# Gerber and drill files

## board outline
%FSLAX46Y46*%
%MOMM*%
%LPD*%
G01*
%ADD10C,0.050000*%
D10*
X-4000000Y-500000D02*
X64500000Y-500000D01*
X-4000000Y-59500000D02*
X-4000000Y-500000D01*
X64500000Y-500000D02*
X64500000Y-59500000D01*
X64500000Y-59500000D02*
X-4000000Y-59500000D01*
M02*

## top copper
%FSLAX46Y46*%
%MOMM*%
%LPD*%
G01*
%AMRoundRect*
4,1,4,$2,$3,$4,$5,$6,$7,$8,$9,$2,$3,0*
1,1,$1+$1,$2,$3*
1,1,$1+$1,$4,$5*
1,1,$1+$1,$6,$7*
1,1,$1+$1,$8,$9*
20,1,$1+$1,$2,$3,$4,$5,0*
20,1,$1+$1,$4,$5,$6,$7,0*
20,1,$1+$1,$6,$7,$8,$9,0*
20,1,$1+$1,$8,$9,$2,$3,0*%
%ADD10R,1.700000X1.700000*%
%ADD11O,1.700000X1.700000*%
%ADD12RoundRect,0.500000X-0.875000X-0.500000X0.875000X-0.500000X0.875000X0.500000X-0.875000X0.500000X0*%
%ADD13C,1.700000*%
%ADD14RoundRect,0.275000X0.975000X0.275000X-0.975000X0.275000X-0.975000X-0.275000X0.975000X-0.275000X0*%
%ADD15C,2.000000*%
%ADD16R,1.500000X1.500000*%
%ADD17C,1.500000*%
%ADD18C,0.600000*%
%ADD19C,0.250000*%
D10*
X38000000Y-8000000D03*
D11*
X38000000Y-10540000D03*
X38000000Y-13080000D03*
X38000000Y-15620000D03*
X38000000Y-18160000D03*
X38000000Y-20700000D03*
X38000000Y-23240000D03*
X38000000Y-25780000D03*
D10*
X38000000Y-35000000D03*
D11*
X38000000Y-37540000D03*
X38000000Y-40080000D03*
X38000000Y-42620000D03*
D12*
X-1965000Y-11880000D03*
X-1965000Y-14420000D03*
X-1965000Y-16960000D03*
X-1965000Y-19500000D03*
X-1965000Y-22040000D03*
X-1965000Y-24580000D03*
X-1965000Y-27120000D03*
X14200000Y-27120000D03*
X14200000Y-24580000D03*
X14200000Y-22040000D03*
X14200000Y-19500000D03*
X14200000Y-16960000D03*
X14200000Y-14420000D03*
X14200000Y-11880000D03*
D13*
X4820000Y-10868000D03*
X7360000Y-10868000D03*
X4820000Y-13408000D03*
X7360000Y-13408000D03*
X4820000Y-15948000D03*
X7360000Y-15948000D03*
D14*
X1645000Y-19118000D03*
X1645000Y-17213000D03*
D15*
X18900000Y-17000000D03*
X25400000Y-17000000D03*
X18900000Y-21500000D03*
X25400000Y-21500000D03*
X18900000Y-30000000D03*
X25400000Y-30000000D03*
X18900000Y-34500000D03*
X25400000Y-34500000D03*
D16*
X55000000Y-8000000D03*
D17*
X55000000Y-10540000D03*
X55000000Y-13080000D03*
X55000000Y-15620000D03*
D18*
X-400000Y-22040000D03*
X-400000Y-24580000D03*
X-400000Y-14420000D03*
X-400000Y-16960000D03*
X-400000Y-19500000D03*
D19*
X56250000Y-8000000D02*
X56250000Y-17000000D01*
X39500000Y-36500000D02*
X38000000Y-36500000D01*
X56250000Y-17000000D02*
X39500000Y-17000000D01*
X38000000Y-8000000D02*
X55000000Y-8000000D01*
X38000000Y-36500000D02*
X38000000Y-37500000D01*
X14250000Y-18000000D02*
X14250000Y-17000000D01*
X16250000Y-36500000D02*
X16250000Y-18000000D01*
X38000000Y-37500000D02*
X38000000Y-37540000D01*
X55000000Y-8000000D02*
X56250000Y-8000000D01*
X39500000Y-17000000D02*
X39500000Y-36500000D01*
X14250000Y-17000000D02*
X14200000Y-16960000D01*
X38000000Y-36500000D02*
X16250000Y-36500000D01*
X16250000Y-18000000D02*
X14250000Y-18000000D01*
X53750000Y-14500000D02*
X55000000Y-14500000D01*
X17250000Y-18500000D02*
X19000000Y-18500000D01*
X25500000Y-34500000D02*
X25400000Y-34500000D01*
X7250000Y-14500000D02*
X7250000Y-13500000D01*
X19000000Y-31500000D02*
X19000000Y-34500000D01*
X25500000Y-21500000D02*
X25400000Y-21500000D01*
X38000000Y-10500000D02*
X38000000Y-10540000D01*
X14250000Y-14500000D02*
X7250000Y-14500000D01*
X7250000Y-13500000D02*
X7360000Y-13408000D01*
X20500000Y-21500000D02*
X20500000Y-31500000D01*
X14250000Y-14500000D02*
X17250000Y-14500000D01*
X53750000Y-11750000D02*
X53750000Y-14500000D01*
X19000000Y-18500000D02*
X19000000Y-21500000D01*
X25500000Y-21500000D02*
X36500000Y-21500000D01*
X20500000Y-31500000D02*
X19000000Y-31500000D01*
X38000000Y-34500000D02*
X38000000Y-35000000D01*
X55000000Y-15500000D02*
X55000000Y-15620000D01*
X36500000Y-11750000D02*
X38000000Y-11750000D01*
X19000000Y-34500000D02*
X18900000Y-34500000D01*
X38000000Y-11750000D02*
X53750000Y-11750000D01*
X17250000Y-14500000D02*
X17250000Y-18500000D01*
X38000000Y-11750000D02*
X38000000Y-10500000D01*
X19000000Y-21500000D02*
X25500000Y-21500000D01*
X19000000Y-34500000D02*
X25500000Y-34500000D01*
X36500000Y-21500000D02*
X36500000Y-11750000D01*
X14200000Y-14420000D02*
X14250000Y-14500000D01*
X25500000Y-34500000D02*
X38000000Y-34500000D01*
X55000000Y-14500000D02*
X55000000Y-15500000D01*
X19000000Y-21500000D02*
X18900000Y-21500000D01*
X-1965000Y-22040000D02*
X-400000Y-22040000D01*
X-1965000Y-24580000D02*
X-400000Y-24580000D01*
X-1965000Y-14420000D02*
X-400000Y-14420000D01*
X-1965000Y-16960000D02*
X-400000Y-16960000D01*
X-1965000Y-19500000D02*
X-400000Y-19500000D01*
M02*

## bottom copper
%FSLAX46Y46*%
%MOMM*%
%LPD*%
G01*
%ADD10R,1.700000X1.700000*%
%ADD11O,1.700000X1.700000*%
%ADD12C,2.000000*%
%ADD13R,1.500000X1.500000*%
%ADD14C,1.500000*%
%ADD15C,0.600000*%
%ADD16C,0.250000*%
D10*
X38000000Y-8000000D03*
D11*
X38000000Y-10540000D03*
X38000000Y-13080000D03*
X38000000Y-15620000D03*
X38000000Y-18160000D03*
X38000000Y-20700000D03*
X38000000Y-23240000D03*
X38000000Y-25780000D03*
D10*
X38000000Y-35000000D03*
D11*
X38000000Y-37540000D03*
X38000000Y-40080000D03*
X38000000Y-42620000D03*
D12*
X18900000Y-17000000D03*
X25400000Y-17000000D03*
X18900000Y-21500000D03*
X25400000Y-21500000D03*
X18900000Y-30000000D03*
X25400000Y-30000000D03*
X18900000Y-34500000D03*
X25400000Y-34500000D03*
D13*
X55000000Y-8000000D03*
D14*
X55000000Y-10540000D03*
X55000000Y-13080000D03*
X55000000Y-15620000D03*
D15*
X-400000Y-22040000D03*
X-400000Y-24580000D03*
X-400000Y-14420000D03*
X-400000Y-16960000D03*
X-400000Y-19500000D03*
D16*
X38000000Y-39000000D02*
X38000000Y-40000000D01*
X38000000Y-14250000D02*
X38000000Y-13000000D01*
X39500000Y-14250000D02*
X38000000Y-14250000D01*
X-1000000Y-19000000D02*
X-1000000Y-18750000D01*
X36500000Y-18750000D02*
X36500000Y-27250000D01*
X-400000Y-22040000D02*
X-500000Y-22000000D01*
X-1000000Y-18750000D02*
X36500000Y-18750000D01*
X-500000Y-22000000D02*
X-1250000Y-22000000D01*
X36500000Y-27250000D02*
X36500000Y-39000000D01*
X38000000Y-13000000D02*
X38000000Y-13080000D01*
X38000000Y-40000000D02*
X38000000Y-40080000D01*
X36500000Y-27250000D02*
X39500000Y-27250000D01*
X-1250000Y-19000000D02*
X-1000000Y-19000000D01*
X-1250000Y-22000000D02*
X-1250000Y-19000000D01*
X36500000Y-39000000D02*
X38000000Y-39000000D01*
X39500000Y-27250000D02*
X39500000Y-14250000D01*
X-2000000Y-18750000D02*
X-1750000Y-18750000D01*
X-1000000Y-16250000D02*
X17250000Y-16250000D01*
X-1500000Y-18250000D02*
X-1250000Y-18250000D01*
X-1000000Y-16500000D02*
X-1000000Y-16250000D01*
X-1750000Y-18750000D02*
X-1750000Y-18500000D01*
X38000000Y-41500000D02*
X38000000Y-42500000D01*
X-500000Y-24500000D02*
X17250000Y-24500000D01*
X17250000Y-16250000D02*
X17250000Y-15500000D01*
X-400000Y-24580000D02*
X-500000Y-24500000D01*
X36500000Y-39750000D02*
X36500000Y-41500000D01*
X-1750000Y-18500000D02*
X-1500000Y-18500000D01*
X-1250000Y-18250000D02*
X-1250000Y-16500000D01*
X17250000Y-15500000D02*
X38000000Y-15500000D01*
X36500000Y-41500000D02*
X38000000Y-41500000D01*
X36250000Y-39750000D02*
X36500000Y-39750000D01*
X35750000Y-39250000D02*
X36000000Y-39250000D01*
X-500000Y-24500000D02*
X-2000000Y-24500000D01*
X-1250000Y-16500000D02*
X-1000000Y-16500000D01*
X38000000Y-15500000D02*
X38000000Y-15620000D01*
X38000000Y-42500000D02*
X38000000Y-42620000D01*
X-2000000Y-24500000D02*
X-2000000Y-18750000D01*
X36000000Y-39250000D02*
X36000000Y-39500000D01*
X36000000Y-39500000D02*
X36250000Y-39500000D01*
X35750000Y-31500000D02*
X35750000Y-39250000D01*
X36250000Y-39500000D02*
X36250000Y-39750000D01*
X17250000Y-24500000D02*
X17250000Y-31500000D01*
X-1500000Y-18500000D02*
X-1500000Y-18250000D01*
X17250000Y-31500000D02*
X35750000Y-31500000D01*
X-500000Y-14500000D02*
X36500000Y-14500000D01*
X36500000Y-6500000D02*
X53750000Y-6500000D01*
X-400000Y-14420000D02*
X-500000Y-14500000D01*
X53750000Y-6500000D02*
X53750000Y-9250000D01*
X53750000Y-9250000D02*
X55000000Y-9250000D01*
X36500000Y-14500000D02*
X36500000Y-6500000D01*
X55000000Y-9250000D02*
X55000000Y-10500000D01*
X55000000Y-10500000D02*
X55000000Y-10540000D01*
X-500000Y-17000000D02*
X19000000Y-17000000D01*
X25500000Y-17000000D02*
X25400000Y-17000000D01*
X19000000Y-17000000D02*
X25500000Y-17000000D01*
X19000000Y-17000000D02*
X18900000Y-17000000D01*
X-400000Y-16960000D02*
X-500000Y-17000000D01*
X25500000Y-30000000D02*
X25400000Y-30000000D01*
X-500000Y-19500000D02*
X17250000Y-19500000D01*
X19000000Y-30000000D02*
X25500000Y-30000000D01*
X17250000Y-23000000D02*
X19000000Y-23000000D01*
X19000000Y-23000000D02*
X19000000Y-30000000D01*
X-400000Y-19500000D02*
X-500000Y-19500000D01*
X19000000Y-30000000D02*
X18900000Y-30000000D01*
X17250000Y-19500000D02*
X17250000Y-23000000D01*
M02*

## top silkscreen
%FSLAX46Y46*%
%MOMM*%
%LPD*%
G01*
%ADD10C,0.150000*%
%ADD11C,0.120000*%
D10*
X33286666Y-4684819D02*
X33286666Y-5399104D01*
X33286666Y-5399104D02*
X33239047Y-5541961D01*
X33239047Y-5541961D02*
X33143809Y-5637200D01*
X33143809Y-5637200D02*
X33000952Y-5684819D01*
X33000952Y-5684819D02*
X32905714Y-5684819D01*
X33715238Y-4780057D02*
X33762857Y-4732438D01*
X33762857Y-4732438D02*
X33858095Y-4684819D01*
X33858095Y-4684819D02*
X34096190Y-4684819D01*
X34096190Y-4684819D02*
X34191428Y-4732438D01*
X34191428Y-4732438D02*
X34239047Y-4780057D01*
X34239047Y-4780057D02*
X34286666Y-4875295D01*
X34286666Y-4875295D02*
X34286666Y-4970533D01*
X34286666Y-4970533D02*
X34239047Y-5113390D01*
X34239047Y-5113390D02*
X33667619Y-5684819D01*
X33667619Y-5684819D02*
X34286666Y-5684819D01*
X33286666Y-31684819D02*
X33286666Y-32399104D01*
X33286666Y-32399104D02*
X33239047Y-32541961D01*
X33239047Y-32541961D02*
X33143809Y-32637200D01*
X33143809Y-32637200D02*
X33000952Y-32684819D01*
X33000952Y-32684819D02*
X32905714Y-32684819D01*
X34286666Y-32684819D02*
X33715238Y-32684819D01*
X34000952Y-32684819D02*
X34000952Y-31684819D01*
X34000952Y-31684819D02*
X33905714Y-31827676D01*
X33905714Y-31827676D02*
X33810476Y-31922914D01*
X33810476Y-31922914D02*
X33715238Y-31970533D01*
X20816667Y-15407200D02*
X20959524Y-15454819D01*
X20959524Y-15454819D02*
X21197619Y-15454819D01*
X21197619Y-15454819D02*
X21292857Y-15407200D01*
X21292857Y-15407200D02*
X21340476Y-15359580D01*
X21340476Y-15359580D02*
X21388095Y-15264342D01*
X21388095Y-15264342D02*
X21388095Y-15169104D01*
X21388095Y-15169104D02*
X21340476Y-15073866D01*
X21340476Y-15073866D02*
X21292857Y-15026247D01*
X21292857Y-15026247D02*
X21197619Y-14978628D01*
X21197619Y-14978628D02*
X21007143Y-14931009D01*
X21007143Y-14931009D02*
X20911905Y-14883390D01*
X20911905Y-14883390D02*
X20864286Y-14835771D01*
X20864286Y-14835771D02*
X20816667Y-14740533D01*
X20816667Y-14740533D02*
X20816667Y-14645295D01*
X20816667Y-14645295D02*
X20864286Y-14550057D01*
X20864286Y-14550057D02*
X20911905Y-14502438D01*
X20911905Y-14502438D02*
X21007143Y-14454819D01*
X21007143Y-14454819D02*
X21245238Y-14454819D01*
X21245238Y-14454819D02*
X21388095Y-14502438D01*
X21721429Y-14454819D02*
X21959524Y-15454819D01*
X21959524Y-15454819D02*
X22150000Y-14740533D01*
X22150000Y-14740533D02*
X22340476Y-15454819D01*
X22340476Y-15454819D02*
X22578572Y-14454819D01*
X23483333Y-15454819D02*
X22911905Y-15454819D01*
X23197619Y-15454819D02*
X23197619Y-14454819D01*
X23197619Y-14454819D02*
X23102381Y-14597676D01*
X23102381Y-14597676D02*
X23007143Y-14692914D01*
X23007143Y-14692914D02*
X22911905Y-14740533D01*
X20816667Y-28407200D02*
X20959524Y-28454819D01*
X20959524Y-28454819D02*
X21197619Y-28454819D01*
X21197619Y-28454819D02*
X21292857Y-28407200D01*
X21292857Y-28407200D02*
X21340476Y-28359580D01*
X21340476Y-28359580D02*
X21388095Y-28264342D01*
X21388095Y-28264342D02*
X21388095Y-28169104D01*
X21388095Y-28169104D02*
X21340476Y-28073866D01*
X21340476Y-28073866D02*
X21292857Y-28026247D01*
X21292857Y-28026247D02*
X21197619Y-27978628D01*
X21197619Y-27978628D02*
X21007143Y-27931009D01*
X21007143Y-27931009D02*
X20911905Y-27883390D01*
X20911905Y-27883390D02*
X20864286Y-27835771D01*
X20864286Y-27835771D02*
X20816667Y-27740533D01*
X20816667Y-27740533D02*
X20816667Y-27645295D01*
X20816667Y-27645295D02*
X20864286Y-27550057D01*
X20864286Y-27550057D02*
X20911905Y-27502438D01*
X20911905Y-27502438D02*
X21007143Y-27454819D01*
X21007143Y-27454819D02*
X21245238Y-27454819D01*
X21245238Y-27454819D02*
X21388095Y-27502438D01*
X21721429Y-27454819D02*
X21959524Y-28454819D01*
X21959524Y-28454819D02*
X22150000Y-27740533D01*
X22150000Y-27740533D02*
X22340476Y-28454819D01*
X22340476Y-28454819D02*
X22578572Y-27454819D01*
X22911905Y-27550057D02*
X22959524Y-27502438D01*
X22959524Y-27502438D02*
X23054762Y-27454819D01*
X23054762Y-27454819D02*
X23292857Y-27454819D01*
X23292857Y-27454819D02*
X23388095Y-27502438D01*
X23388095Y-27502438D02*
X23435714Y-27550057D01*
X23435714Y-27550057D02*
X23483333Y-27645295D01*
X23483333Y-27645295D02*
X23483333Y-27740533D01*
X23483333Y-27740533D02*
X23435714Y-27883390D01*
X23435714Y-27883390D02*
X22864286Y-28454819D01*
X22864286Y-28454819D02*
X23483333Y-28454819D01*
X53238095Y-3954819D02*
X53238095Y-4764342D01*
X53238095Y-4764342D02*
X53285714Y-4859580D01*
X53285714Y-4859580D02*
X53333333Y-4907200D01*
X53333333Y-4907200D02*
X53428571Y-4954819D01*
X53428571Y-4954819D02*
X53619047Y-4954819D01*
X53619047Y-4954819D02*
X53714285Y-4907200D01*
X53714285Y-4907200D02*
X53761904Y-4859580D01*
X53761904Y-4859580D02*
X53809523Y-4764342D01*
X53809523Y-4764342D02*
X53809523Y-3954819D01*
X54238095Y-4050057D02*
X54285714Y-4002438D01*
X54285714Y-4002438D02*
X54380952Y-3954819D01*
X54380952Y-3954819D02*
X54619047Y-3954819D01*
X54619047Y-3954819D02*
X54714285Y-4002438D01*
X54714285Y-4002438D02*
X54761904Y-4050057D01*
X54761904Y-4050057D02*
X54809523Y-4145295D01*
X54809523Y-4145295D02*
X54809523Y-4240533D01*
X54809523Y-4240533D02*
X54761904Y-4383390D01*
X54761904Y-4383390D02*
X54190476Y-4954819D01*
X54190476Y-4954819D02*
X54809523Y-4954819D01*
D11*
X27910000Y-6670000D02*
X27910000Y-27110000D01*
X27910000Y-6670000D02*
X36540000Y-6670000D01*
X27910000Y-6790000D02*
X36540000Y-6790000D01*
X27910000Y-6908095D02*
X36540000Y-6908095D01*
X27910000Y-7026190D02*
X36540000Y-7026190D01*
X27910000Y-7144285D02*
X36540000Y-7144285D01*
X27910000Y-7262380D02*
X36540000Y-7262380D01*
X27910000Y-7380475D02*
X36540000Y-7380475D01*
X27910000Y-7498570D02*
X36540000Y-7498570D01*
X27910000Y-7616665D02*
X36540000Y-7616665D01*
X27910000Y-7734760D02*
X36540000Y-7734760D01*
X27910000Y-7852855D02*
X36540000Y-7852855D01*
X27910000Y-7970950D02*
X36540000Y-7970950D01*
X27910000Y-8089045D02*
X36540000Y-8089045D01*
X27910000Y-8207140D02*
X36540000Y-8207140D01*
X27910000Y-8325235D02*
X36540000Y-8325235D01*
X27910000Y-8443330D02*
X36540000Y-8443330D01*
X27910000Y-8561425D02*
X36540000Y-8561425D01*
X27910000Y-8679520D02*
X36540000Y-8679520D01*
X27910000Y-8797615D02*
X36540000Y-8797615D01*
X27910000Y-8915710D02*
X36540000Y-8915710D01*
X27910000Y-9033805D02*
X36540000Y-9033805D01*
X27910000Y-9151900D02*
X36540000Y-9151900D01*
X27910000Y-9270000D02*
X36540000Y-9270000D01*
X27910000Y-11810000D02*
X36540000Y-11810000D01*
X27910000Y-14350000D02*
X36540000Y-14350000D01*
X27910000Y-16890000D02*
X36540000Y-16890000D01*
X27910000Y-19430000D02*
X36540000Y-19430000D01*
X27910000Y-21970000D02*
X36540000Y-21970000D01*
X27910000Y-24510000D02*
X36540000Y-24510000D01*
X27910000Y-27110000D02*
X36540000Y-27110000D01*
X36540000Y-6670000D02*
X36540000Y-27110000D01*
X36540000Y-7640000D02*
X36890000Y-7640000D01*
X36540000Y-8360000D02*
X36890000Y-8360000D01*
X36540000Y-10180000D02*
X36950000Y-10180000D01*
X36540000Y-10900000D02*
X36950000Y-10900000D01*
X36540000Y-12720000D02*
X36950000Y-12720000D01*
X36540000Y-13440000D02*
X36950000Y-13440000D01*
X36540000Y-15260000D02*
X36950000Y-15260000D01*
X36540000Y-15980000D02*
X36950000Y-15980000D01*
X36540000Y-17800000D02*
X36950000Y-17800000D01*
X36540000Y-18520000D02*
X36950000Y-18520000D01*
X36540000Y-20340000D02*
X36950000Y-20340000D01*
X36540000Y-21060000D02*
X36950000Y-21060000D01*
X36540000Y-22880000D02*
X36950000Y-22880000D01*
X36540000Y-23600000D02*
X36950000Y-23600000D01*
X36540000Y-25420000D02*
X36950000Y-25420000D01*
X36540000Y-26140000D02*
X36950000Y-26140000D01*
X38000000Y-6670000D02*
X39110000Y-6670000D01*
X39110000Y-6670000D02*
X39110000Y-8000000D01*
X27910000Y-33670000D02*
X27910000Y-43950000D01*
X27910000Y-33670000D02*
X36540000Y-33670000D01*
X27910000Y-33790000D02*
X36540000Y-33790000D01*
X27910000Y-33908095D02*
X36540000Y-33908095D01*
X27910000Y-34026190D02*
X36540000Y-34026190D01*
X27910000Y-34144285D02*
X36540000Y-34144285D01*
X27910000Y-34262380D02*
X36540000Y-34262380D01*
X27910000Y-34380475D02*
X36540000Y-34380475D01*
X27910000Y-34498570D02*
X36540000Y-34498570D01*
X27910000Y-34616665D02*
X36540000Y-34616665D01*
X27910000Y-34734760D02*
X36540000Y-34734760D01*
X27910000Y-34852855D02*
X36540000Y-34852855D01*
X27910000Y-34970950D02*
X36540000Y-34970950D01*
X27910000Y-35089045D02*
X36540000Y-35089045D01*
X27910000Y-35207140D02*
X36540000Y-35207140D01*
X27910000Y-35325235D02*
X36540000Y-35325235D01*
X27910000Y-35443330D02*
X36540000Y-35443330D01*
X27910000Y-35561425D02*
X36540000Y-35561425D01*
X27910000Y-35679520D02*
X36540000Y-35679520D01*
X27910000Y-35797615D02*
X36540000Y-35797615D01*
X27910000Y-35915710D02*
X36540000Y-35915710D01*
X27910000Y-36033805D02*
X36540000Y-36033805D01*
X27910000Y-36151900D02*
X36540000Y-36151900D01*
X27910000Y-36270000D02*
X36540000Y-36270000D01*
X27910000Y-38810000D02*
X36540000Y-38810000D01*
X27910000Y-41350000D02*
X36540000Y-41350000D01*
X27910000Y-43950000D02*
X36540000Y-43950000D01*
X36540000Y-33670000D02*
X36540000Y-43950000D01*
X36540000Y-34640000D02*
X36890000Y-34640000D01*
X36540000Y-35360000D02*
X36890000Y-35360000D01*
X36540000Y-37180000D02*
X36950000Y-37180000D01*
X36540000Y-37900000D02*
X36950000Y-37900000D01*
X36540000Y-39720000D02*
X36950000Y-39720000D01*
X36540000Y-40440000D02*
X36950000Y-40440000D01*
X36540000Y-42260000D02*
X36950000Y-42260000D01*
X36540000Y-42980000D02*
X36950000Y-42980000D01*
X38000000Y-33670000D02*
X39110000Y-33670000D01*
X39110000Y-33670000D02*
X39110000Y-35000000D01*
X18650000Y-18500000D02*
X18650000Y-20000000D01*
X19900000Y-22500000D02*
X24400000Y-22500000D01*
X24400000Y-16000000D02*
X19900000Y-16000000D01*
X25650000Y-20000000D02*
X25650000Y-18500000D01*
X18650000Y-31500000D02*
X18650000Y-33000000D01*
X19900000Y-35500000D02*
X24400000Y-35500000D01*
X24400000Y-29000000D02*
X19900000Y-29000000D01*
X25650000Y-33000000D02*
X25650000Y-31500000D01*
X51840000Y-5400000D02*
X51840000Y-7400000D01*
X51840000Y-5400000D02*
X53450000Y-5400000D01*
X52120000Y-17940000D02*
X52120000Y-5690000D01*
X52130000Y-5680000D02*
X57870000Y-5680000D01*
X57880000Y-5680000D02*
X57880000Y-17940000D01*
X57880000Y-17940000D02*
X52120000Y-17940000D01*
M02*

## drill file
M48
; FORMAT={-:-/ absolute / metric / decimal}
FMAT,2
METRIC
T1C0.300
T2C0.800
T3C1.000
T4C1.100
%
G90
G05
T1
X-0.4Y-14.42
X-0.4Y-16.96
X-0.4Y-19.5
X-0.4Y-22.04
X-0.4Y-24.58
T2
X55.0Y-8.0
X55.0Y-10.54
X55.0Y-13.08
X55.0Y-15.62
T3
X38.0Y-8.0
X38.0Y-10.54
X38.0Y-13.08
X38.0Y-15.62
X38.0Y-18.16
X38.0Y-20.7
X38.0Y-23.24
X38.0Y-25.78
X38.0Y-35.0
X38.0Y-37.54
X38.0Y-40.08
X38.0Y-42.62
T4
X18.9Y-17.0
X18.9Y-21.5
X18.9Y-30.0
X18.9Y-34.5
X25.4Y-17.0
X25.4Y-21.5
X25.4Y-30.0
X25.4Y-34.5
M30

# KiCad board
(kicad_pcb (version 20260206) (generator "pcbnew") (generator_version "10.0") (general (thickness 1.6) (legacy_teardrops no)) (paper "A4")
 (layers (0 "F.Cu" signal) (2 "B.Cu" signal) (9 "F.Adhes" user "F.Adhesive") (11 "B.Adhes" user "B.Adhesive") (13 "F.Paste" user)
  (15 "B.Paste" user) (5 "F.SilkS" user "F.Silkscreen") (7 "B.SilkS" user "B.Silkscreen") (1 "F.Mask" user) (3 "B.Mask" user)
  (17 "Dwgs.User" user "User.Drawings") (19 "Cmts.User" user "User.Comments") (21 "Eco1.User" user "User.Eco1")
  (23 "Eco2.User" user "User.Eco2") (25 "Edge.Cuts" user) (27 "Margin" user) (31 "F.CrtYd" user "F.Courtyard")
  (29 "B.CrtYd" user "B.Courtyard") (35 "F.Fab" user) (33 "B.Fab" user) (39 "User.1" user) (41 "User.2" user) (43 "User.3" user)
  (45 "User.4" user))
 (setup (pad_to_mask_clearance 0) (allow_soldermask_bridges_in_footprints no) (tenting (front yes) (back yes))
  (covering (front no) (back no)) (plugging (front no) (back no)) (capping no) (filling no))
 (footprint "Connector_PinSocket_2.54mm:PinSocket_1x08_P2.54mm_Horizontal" (layer "F.Cu") (at 38 8)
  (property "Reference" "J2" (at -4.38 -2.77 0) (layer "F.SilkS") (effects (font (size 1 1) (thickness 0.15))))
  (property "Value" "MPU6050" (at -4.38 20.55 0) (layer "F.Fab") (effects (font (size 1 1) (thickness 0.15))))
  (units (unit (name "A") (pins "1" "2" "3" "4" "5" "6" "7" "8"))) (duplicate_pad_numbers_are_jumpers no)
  (fp_line (start -10.09 -1.33) (end -10.09 19.11) (stroke (width 0.12) (type solid)) (layer "F.SilkS"))
  (fp_line (start -10.09 -1.33) (end -1.46 -1.33) (stroke (width 0.12) (type solid)) (layer "F.SilkS"))
  (fp_line (start -10.09 -1.21) (end -1.46 -1.21) (stroke (width 0.12) (type solid)) (layer "F.SilkS"))
  (fp_line (start -10.09 -1.091905) (end -1.46 -1.091905) (stroke (width 0.12) (type solid)) (layer "F.SilkS"))
  (fp_line (start -10.09 -0.97381) (end -1.46 -0.97381) (stroke (width 0.12) (type solid)) (layer "F.SilkS"))
  (fp_line (start -10.09 -0.855715) (end -1.46 -0.855715) (stroke (width 0.12) (type solid)) (layer "F.SilkS"))
  (fp_line (start -10.09 -0.73762) (end -1.46 -0.73762) (stroke (width 0.12) (type solid)) (layer "F.SilkS"))
  (fp_line (start -10.09 -0.619525) (end -1.46 -0.619525) (stroke (width 0.12) (type solid)) (layer "F.SilkS"))
  (fp_line (start -10.09 -0.50143) (end -1.46 -0.50143) (stroke (width 0.12) (type solid)) (layer "F.SilkS"))
  (fp_line (start -10.09 -0.383335) (end -1.46 -0.383335) (stroke (width 0.12) (type solid)) (layer "F.SilkS"))
  (fp_line (start -10.09 -0.26524) (end -1.46 -0.26524) (stroke (width 0.12) (type solid)) (layer "F.SilkS"))
  (fp_line (start -10.09 -0.147145) (end -1.46 -0.147145) (stroke (width 0.12) (type solid)) (layer "F.SilkS"))
  (fp_line (start -10.09 -0.02905) (end -1.46 -0.02905) (stroke (width 0.12) (type solid)) (layer "F.SilkS"))
  (fp_line (start -10.09 0.089045) (end -1.46 0.089045) (stroke (width 0.12) (type solid)) (layer "F.SilkS"))
  (fp_line (start -10.09 0.20714) (end -1.46 0.20714) (stroke (width 0.12) (type solid)) (layer "F.SilkS"))
  (fp_line (start -10.09 0.325235) (end -1.46 0.325235) (stroke (width 0.12) (type solid)) (layer "F.SilkS"))
  (fp_line (start -10.09 0.44333) (end -1.46 0.44333) (stroke (width 0.12) (type solid)) (layer "F.SilkS"))
  (fp_line (start -10.09 0.561425) (end -1.46 0.561425) (stroke (width 0.12) (type solid)) (layer "F.SilkS"))
  (fp_line (start -10.09 0.67952) (end -1.46 0.67952) (stroke (width 0.12) (type solid)) (layer "F.SilkS"))
  (fp_line (start -10.09 0.797615) (end -1.46 0.797615) (stroke (width 0.12) (type solid)) (layer "F.SilkS"))
  (fp_line (start -10.09 0.91571) (end -1.46 0.91571) (stroke (width 0.12) (type solid)) (layer "F.SilkS"))
  (fp_line (start -10.09 1.033805) (end -1.46 1.033805) (stroke (width 0.12) (type solid)) (layer "F.SilkS"))
  (fp_line (start -10.09 1.1519) (end -1.46 1.1519) (stroke (width 0.12) (type solid)) (layer "F.SilkS"))
  (fp_line (start -10.09 1.27) (end -1.46 1.27) (stroke (width 0.12) (type solid)) (layer "F.SilkS"))
  (fp_line (start -10.09 3.81) (end -1.46 3.81) (stroke (width 0.12) (type solid)) (layer "F.SilkS"))
  (fp_line (start -10.09 6.35) (end -1.46 6.35) (stroke (width 0.12) (type solid)) (layer "F.SilkS"))
  (fp_line (start -10.09 8.89) (end -1.46 8.89) (stroke (width 0.12) (type solid)) (layer "F.SilkS"))
  (fp_line (start -10.09 11.43) (end -1.46 11.43) (stroke (width 0.12) (type solid)) (layer "F.SilkS"))
  (fp_line (start -10.09 13.97) (end -1.46 13.97) (stroke (width 0.12) (type solid)) (layer "F.SilkS"))
  (fp_line (start -10.09 16.51) (end -1.46 16.51) (stroke (width 0.12) (type solid)) (layer "F.SilkS"))
  (fp_line (start -10.09 19.11) (end -1.46 19.11) (stroke (width 0.12) (type solid)) (layer "F.SilkS"))
  (fp_line (start -1.46 -1.33) (end -1.46 19.11) (stroke (width 0.12) (type solid)) (layer "F.SilkS"))
  (fp_line (start -1.46 -0.36) (end -1.11 -0.36) (stroke (width 0.12) (type solid)) (layer "F.SilkS"))
  (fp_line (start -1.46 0.36) (end -1.11 0.36) (stroke (width 0.12) (type solid)) (layer "F.SilkS"))
  (fp_line (start -1.46 2.18) (end -1.05 2.18) (stroke (width 0.12) (type solid)) (layer "F.SilkS"))
  (fp_line (start -1.46 2.9) (end -1.05 2.9) (stroke (width 0.12) (type solid)) (layer "F.SilkS"))
  (fp_line (start -1.46 4.72) (end -1.05 4.72) (stroke (width 0.12) (type solid)) (layer "F.SilkS"))
  (fp_line (start -1.46 5.44) (end -1.05 5.44) (stroke (width 0.12) (type solid)) (layer "F.SilkS"))
  (fp_line (start -1.46 7.26) (end -1.05 7.26) (stroke (width 0.12) (type solid)) (layer "F.SilkS"))
  (fp_line (start -1.46 7.98) (end -1.05 7.98) (stroke (width 0.12) (type solid)) (layer "F.SilkS"))
  (fp_line (start -1.46 9.8) (end -1.05 9.8) (stroke (width 0.12) (type solid)) (layer "F.SilkS"))
  (fp_line (start -1.46 10.52) (end -1.05 10.52) (stroke (width 0.12) (type solid)) (layer "F.SilkS"))
  (fp_line (start -1.46 12.34) (end -1.05 12.34) (stroke (width 0.12) (type solid)) (layer "F.SilkS"))
  (fp_line (start -1.46 13.06) (end -1.05 13.06) (stroke (width 0.12) (type solid)) (layer "F.SilkS"))
  (fp_line (start -1.46 14.88) (end -1.05 14.88) (stroke (width 0.12) (type solid)) (layer "F.SilkS"))
  (fp_line (start -1.46 15.6) (end -1.05 15.6) (stroke (width 0.12) (type solid)) (layer "F.SilkS"))
  (fp_line (start -1.46 17.42) (end -1.05 17.42) (stroke (width 0.12) (type solid)) (layer "F.SilkS"))
  (fp_line (start -1.46 18.14) (end -1.05 18.14) (stroke (width 0.12) (type solid)) (layer "F.SilkS"))
  (fp_line (start 0 -1.33) (end 1.11 -1.33) (stroke (width 0.12) (type solid)) (layer "F.SilkS"))
  (fp_line (start 1.11 -1.33) (end 1.11 0) (stroke (width 0.12) (type solid)) (layer "F.SilkS"))
  (pad "1" thru_hole rect (at 0 0) (size 1.7 1.7) (drill 1) (layers "*.Cu" "*.Mask") (remove_unused_layers no) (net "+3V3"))
  (pad "2" thru_hole oval (at 0 2.54) (size 1.7 1.7) (drill 1) (layers "*.Cu" "*.Mask") (remove_unused_layers no) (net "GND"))
  (pad "3" thru_hole oval (at 0 5.08) (size 1.7 1.7) (drill 1) (layers "*.Cu" "*.Mask") (remove_unused_layers no) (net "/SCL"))
  (pad "4" thru_hole oval (at 0 7.62) (size 1.7 1.7) (drill 1) (layers "*.Cu" "*.Mask") (remove_unused_layers no) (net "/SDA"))
  (pad "5" thru_hole oval (at 0 10.16) (size 1.7 1.7) (drill 1) (layers "*.Cu" "*.Mask") (remove_unused_layers no)
   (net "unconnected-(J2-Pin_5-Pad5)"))
  (pad "6" thru_hole oval (at 0 12.7) (size 1.7 1.7) (drill 1) (layers "*.Cu" "*.Mask") (remove_unused_layers no)
   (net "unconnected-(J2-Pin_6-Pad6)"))
  (pad "7" thru_hole oval (at 0 15.24) (size 1.7 1.7) (drill 1) (layers "*.Cu" "*.Mask") (remove_unused_layers no)
   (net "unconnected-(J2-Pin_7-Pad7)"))
  (pad "8" thru_hole oval (at 0 17.78) (size 1.7 1.7) (drill 1) (layers "*.Cu" "*.Mask") (remove_unused_layers no)
   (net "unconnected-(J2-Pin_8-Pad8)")))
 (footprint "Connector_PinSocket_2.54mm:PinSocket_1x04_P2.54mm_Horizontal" (layer "F.Cu") (at 38 35)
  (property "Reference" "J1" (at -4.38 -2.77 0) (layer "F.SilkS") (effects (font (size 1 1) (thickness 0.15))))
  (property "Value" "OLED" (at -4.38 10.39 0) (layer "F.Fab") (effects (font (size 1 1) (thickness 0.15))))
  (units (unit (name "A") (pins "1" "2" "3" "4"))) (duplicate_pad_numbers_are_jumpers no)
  (fp_line (start -10.09 -1.33) (end -10.09 8.95) (stroke (width 0.12) (type solid)) (layer "F.SilkS"))
  (fp_line (start -10.09 -1.33) (end -1.46 -1.33) (stroke (width 0.12) (type solid)) (layer "F.SilkS"))
  (fp_line (start -10.09 -1.21) (end -1.46 -1.21) (stroke (width 0.12) (type solid)) (layer "F.SilkS"))
  (fp_line (start -10.09 -1.091905) (end -1.46 -1.091905) (stroke (width 0.12) (type solid)) (layer "F.SilkS"))
  (fp_line (start -10.09 -0.97381) (end -1.46 -0.97381) (stroke (width 0.12) (type solid)) (layer "F.SilkS"))
  (fp_line (start -10.09 -0.855715) (end -1.46 -0.855715) (stroke (width 0.12) (type solid)) (layer "F.SilkS"))
  (fp_line (start -10.09 -0.73762) (end -1.46 -0.73762) (stroke (width 0.12) (type solid)) (layer "F.SilkS"))
  (fp_line (start -10.09 -0.619525) (end -1.46 -0.619525) (stroke (width 0.12) (type solid)) (layer "F.SilkS"))
  (fp_line (start -10.09 -0.50143) (end -1.46 -0.50143) (stroke (width 0.12) (type solid)) (layer "F.SilkS"))
  (fp_line (start -10.09 -0.383335) (end -1.46 -0.383335) (stroke (width 0.12) (type solid)) (layer "F.SilkS"))
  (fp_line (start -10.09 -0.26524) (end -1.46 -0.26524) (stroke (width 0.12) (type solid)) (layer "F.SilkS"))
  (fp_line (start -10.09 -0.147145) (end -1.46 -0.147145) (stroke (width 0.12) (type solid)) (layer "F.SilkS"))
  (fp_line (start -10.09 -0.02905) (end -1.46 -0.02905) (stroke (width 0.12) (type solid)) (layer "F.SilkS"))
  (fp_line (start -10.09 0.089045) (end -1.46 0.089045) (stroke (width 0.12) (type solid)) (layer "F.SilkS"))
  (fp_line (start -10.09 0.20714) (end -1.46 0.20714) (stroke (width 0.12) (type solid)) (layer "F.SilkS"))
  (fp_line (start -10.09 0.325235) (end -1.46 0.325235) (stroke (width 0.12) (type solid)) (layer "F.SilkS"))
  (fp_line (start -10.09 0.44333) (end -1.46 0.44333) (stroke (width 0.12) (type solid)) (layer "F.SilkS"))
  (fp_line (start -10.09 0.561425) (end -1.46 0.561425) (stroke (width 0.12) (type solid)) (layer "F.SilkS"))
  (fp_line (start -10.09 0.67952) (end -1.46 0.67952) (stroke (width 0.12) (type solid)) (layer "F.SilkS"))
  (fp_line (start -10.09 0.797615) (end -1.46 0.797615) (stroke (width 0.12) (type solid)) (layer "F.SilkS"))
  (fp_line (start -10.09 0.91571) (end -1.46 0.91571) (stroke (width 0.12) (type solid)) (layer "F.SilkS"))
  (fp_line (start -10.09 1.033805) (end -1.46 1.033805) (stroke (width 0.12) (type solid)) (layer "F.SilkS"))
  (fp_line (start -10.09 1.1519) (end -1.46 1.1519) (stroke (width 0.12) (type solid)) (layer "F.SilkS"))
  (fp_line (start -10.09 1.27) (end -1.46 1.27) (stroke (width 0.12) (type solid)) (layer "F.SilkS"))
  (fp_line (start -10.09 3.81) (end -1.46 3.81) (stroke (width 0.12) (type solid)) (layer "F.SilkS"))
  (fp_line (start -10.09 6.35) (end -1.46 6.35) (stroke (width 0.12) (type solid)) (layer "F.SilkS"))
  (fp_line (start -10.09 8.95) (end -1.46 8.95) (stroke (width 0.12) (type solid)) (layer "F.SilkS"))
  (fp_line (start -1.46 -1.33) (end -1.46 8.95) (stroke (width 0.12) (type solid)) (layer "F.SilkS"))
  (fp_line (start -1.46 -0.36) (end -1.11 -0.36) (stroke (width 0.12) (type solid)) (layer "F.SilkS"))
  (fp_line (start -1.46 0.36) (end -1.11 0.36) (stroke (width 0.12) (type solid)) (layer "F.SilkS"))
  (fp_line (start -1.46 2.18) (end -1.05 2.18) (stroke (width 0.12) (type solid)) (layer "F.SilkS"))
  (fp_line (start -1.46 2.9) (end -1.05 2.9) (stroke (width 0.12) (type solid)) (layer "F.SilkS"))
  (fp_line (start -1.46 4.72) (end -1.05 4.72) (stroke (width 0.12) (type solid)) (layer "F.SilkS"))
  (fp_line (start -1.46 5.44) (end -1.05 5.44) (stroke (width 0.12) (type solid)) (layer "F.SilkS"))
  (fp_line (start -1.46 7.26) (end -1.05 7.26) (stroke (width 0.12) (type solid)) (layer "F.SilkS"))
  (fp_line (start -1.46 7.98) (end -1.05 7.98) (stroke (width 0.12) (type solid)) (layer "F.SilkS"))
  (fp_line (start 0 -1.33) (end 1.11 -1.33) (stroke (width 0.12) (type solid)) (layer "F.SilkS"))
  (fp_line (start 1.11 -1.33) (end 1.11 0) (stroke (width 0.12) (type solid)) (layer "F.SilkS"))
  (pad "1" thru_hole rect (at 0 0) (size 1.7 1.7) (drill 1) (layers "*.Cu" "*.Mask") (remove_unused_layers no) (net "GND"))
  (pad "2" thru_hole oval (at 0 2.54) (size 1.7 1.7) (drill 1) (layers "*.Cu" "*.Mask") (remove_unused_layers no) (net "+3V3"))
  (pad "3" thru_hole oval (at 0 5.08) (size 1.7 1.7) (drill 1) (layers "*.Cu" "*.Mask") (remove_unused_layers no) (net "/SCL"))
  (pad "4" thru_hole oval (at 0 7.62) (size 1.7 1.7) (drill 1) (layers "*.Cu" "*.Mask") (remove_unused_layers no) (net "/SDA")))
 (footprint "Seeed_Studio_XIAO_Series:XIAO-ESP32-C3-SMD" (layer "F.Cu") (at -2.8 30)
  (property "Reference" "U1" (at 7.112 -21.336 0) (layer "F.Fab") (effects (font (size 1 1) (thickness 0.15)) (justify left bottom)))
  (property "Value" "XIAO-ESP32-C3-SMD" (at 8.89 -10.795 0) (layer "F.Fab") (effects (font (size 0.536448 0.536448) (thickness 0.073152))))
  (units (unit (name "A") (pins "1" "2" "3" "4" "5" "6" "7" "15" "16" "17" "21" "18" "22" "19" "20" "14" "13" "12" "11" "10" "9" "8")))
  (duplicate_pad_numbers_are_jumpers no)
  (pad "1" smd roundrect (at 0.835 -18.12) (size 2.75 2) (layers "F.Cu" "F.Mask" "F.Paste") (roundrect_rratio 0.25)
   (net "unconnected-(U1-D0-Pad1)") (solder_mask_margin 0.0508) (thermal_bridge_angle 45))
  (pad "2" smd roundrect (at 0.835 -15.58) (size 2.75 2) (layers "F.Cu" "F.Mask" "F.Paste") (roundrect_rratio 0.25) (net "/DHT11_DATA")
   (solder_mask_margin 0.0508) (thermal_bridge_angle 45))
  (pad "3" smd roundrect (at 0.835 -13.04) (size 2.75 2) (layers "F.Cu" "F.Mask" "F.Paste") (roundrect_rratio 0.25) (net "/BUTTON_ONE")
   (solder_mask_margin 0.0508) (thermal_bridge_angle 45))
  (pad "4" smd roundrect (at 0.835 -10.5) (size 2.75 2) (layers "F.Cu" "F.Mask" "F.Paste") (roundrect_rratio 0.25) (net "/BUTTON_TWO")
   (solder_mask_margin 0.0508) (thermal_bridge_angle 45))
  (pad "5" smd roundrect (at 0.835 -7.96) (size 2.75 2) (layers "F.Cu" "F.Mask" "F.Paste") (roundrect_rratio 0.25) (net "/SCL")
   (solder_mask_margin 0.0508) (thermal_bridge_angle 45))
  (pad "6" smd roundrect (at 0.835 -5.42) (size 2.75 2) (layers "F.Cu" "F.Mask" "F.Paste") (roundrect_rratio 0.25) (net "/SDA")
   (solder_mask_margin 0.0508) (thermal_bridge_angle 45))
  (pad "7" smd roundrect (at 0.835 -2.88) (size 2.75 2) (layers "F.Cu" "F.Mask" "F.Paste") (roundrect_rratio 0.25)
   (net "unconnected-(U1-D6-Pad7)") (solder_mask_margin 0.0508) (thermal_bridge_angle 45))
  (pad "8" smd roundrect (at 17 -2.88) (size 2.75 2) (layers "F.Cu" "F.Mask" "F.Paste") (roundrect_rratio 0.25)
   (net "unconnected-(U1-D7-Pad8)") (solder_mask_margin 0.0508) (thermal_bridge_angle 45))
  (pad "9" smd roundrect (at 17 -5.42) (size 2.75 2) (layers "F.Cu" "F.Mask" "F.Paste") (roundrect_rratio 0.25)
   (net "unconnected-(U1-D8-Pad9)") (solder_mask_margin 0.0508) (thermal_bridge_angle 45))
  (pad "10" smd roundrect (at 17 -7.96) (size 2.75 2) (layers "F.Cu" "F.Mask" "F.Paste") (roundrect_rratio 0.25)
   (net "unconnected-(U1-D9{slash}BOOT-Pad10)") (solder_mask_margin 0.0508) (thermal_bridge_angle 45))
  (pad "11" smd roundrect (at 17 -10.5) (size 2.75 2) (layers "F.Cu" "F.Mask" "F.Paste") (roundrect_rratio 0.25)
   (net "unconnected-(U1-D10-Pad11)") (solder_mask_margin 0.0508) (thermal_bridge_angle 45))
  (pad "12" smd roundrect (at 17 -13.04) (size 2.75 2) (layers "F.Cu" "F.Mask" "F.Paste") (roundrect_rratio 0.25) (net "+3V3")
   (solder_mask_margin 0.0508) (thermal_bridge_angle 45))
  (pad "13" smd roundrect (at 17 -15.58) (size 2.75 2) (layers "F.Cu" "F.Mask" "F.Paste") (roundrect_rratio 0.25) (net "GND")
   (solder_mask_margin 0.0508) (thermal_bridge_angle 45))
  (pad "14" smd roundrect (at 17 -18.12) (size 2.75 2) (layers "F.Cu" "F.Mask" "F.Paste") (roundrect_rratio 0.25) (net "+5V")
   (solder_mask_margin 0.0508) (thermal_bridge_angle 45))
  (pad "15" smd circle (at 7.62 -19.132) (size 1.7 1.7) (layers "F.Cu" "F.Mask" "F.Paste") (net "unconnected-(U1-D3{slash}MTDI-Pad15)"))
  (pad "16" smd circle (at 10.16 -19.132) (size 1.7 1.7) (layers "F.Cu" "F.Mask" "F.Paste") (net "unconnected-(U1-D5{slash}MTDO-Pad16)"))
  (pad "17" smd circle (at 7.62 -16.592) (size 1.7 1.7) (layers "F.Cu" "F.Mask" "F.Paste") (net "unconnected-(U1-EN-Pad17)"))
  (pad "18" smd circle (at 10.16 -16.592) (size 1.7 1.7) (layers "F.Cu" "F.Mask" "F.Paste") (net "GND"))
  (pad "19" smd circle (at 7.62 -14.052) (size 1.7 1.7) (layers "F.Cu" "F.Mask" "F.Paste") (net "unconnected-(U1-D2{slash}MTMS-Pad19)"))
  (pad "20" smd circle (at 10.16 -14.052) (size 1.7 1.7) (layers "F.Cu" "F.Mask" "F.Paste") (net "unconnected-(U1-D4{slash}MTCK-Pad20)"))
  (pad "21" smd roundrect (at 4.445 -10.882 180) (size 2.5 1.1) (layers "F.Cu" "F.Mask" "F.Paste") (roundrect_rratio 0.25)
   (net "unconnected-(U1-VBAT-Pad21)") (thermal_bridge_angle 45))
  (pad "22" smd roundrect (at 4.445 -12.787 180) (size 2.5 1.1) (layers "F.Cu" "F.Mask" "F.Paste") (roundrect_rratio 0.25)
   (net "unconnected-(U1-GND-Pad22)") (thermal_bridge_angle 45)))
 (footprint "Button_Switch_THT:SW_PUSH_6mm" (layer "F.Cu") (at 18.9 17)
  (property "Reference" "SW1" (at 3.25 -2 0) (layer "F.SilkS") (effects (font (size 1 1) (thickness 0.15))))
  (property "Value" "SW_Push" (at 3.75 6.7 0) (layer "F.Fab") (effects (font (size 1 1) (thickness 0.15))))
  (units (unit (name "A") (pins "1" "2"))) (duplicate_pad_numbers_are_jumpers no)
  (fp_line (start -0.25 1.5) (end -0.25 3) (stroke (width 0.12) (type solid)) (layer "F.SilkS"))
  (fp_line (start 1 5.5) (end 5.5 5.5) (stroke (width 0.12) (type solid)) (layer "F.SilkS"))
  (fp_line (start 5.5 -1) (end 1 -1) (stroke (width 0.12) (type solid)) (layer "F.SilkS"))
  (fp_line (start 6.75 3) (end 6.75 1.5) (stroke (width 0.12) (type solid)) (layer "F.SilkS"))
  (pad "1" thru_hole circle (at 0 0 90) (size 2 2) (drill 1.1) (layers "*.Cu" "*.Mask") (remove_unused_layers no) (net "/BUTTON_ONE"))
  (pad "1" thru_hole circle (at 6.5 0 90) (size 2 2) (drill 1.1) (layers "*.Cu" "*.Mask") (remove_unused_layers no) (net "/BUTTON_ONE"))
  (pad "2" thru_hole circle (at 0 4.5 90) (size 2 2) (drill 1.1) (layers "*.Cu" "*.Mask") (remove_unused_layers no) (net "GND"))
  (pad "2" thru_hole circle (at 6.5 4.5 90) (size 2 2) (drill 1.1) (layers "*.Cu" "*.Mask") (remove_unused_layers no) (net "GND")))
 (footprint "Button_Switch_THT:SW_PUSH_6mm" (layer "F.Cu") (at 18.9 30)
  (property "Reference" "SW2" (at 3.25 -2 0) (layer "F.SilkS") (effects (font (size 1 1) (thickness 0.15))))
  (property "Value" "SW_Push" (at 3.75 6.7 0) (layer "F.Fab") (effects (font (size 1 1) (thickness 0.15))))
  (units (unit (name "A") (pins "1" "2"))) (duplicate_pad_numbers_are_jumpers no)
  (fp_line (start -0.25 1.5) (end -0.25 3) (stroke (width 0.12) (type solid)) (layer "F.SilkS"))
  (fp_line (start 1 5.5) (end 5.5 5.5) (stroke (width 0.12) (type solid)) (layer "F.SilkS"))
  (fp_line (start 5.5 -1) (end 1 -1) (stroke (width 0.12) (type solid)) (layer "F.SilkS"))
  (fp_line (start 6.75 3) (end 6.75 1.5) (stroke (width 0.12) (type solid)) (layer "F.SilkS"))
  (pad "1" thru_hole circle (at 0 0 90) (size 2 2) (drill 1.1) (layers "*.Cu" "*.Mask") (remove_unused_layers no) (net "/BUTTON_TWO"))
  (pad "1" thru_hole circle (at 6.5 0 90) (size 2 2) (drill 1.1) (layers "*.Cu" "*.Mask") (remove_unused_layers no) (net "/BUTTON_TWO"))
  (pad "2" thru_hole circle (at 0 4.5 90) (size 2 2) (drill 1.1) (layers "*.Cu" "*.Mask") (remove_unused_layers no) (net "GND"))
  (pad "2" thru_hole circle (at 6.5 4.5 90) (size 2 2) (drill 1.1) (layers "*.Cu" "*.Mask") (remove_unused_layers no) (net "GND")))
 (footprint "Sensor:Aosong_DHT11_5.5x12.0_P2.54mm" (layer "F.Cu") (at 55 8)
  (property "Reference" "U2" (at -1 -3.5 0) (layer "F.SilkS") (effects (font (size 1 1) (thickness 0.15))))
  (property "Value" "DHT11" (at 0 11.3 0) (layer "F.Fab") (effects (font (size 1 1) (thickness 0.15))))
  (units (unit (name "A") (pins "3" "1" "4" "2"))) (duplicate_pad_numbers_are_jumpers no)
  (fp_line (start -3.16 -2.6) (end -3.16 -0.6) (stroke (width 0.12) (type solid)) (layer "F.SilkS"))
  (fp_line (start -3.16 -2.6) (end -1.55 -2.6) (stroke (width 0.12) (type solid)) (layer "F.SilkS"))
  (fp_line (start -2.88 9.94) (end -2.88 -2.31) (stroke (width 0.12) (type solid)) (layer "F.SilkS"))
  (fp_line (start -2.87 -2.32) (end 2.87 -2.32) (stroke (width 0.12) (type solid)) (layer "F.SilkS"))
  (fp_line (start 2.88 -2.32) (end 2.88 9.94) (stroke (width 0.12) (type solid)) (layer "F.SilkS"))
  (fp_line (start 2.88 9.94) (end -2.88 9.94) (stroke (width 0.12) (type solid)) (layer "F.SilkS"))
  (pad "1" thru_hole rect (at 0 0) (size 1.5 1.5) (drill 0.8) (layers "*.Cu" "*.Mask") (remove_unused_layers no) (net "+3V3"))
  (pad "2" thru_hole circle (at 0 2.54) (size 1.5 1.5) (drill 0.8) (layers "*.Cu" "*.Mask") (remove_unused_layers no) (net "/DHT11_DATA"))
  (pad "3" thru_hole circle (at 0 5.08) (size 1.5 1.5) (drill 0.8) (layers "*.Cu" "*.Mask") (remove_unused_layers no)
   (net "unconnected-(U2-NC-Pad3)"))
  (pad "4" thru_hole circle (at 0 7.62) (size 1.5 1.5) (drill 0.8) (layers "*.Cu" "*.Mask") (remove_unused_layers no) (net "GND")))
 (gr_line (start -4 0.5) (end 64.5 0.5) (stroke (width 0.05) (type default)) (layer "Edge.Cuts"))
 (gr_line (start -4 59.5) (end -4 0.5) (stroke (width 0.05) (type default)) (layer "Edge.Cuts"))
 (gr_line (start 64.5 0.5) (end 64.5 59.5) (stroke (width 0.05) (type default)) (layer "Edge.Cuts"))
 (gr_line (start 64.5 59.5) (end -4 59.5) (stroke (width 0.05) (type default)) (layer "Edge.Cuts"))
 (segment (start 56.25 8) (end 56.25 17) (width 0.25) (layer "F.Cu") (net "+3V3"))
 (segment (start 39.5 36.5) (end 38 36.5) (width 0.25) (layer "F.Cu") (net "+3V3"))
 (segment (start 56.25 17) (end 39.5 17) (width 0.25) (layer "F.Cu") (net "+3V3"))
 (segment (start 38 8) (end 55 8) (width 0.25) (layer "F.Cu") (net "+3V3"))
 (segment (start 38 36.5) (end 38 37.5) (width 0.25) (layer "F.Cu") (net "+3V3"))
 (segment (start 14.25 18) (end 14.25 17) (width 0.25) (layer "F.Cu") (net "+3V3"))
 (segment (start 16.25 36.5) (end 16.25 18) (width 0.25) (layer "F.Cu") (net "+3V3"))
 (segment (start 38 37.5) (end 38 37.54) (width 0.25) (layer "F.Cu") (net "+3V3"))
 (segment (start 55 8) (end 56.25 8) (width 0.25) (layer "F.Cu") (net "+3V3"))
 (segment (start 39.5 17) (end 39.5 36.5) (width 0.25) (layer "F.Cu") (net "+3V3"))
 (segment (start 14.25 17) (end 14.2 16.96) (width 0.25) (layer "F.Cu") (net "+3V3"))
 (segment (start 38 36.5) (end 16.25 36.5) (width 0.25) (layer "F.Cu") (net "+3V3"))
 (segment (start 16.25 18) (end 14.25 18) (width 0.25) (layer "F.Cu") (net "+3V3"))
 (segment (start 53.75 14.5) (end 55 14.5) (width 0.25) (layer "F.Cu") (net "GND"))
 (segment (start 17.25 18.5) (end 19 18.5) (width 0.25) (layer "F.Cu") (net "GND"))
 (segment (start 25.5 34.5) (end 25.4 34.5) (width 0.25) (layer "F.Cu") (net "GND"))
 (segment (start 7.25 14.5) (end 7.25 13.5) (width 0.25) (layer "F.Cu") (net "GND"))
 (segment (start 19 31.5) (end 19 34.5) (width 0.25) (layer "F.Cu") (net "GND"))
 (segment (start 25.5 21.5) (end 25.4 21.5) (width 0.25) (layer "F.Cu") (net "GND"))
 (segment (start 38 10.5) (end 38 10.54) (width 0.25) (layer "F.Cu") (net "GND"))
 (segment (start 14.25 14.5) (end 7.25 14.5) (width 0.25) (layer "F.Cu") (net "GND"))
 (segment (start 7.25 13.5) (end 7.36 13.408) (width 0.25) (layer "F.Cu") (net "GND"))
 (segment (start 20.5 21.5) (end 20.5 31.5) (width 0.25) (layer "F.Cu") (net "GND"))
 (segment (start 14.25 14.5) (end 17.25 14.5) (width 0.25) (layer "F.Cu") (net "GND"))
 (segment (start 53.75 11.75) (end 53.75 14.5) (width 0.25) (layer "F.Cu") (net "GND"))
 (segment (start 19 18.5) (end 19 21.5) (width 0.25) (layer "F.Cu") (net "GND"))
 (segment (start 25.5 21.5) (end 36.5 21.5) (width 0.25) (layer "F.Cu") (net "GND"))
 (segment (start 20.5 31.5) (end 19 31.5) (width 0.25) (layer "F.Cu") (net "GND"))
 (segment (start 38 34.5) (end 38 35) (width 0.25) (layer "F.Cu") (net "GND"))
 (segment (start 55 15.5) (end 55 15.62) (width 0.25) (layer "F.Cu") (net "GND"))
 (segment (start 36.5 11.75) (end 38 11.75) (width 0.25) (layer "F.Cu") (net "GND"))
 (segment (start 19 34.5) (end 18.9 34.5) (width 0.25) (layer "F.Cu") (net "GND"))
 (segment (start 38 11.75) (end 53.75 11.75) (width 0.25) (layer "F.Cu") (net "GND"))
 (segment (start 17.25 14.5) (end 17.25 18.5) (width 0.25) (layer "F.Cu") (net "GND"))
 (segment (start 38 11.75) (end 38 10.5) (width 0.25) (layer "F.Cu") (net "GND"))
 (segment (start 19 21.5) (end 25.5 21.5) (width 0.25) (layer "F.Cu") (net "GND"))
 (segment (start 19 34.5) (end 25.5 34.5) (width 0.25) (layer "F.Cu") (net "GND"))
 (segment (start 36.5 21.5) (end 36.5 11.75) (width 0.25) (layer "F.Cu") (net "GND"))
 (segment (start 14.2 14.42) (end 14.25 14.5) (width 0.25) (layer "F.Cu") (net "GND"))
 (segment (start 25.5 34.5) (end 38 34.5) (width 0.25) (layer "F.Cu") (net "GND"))
 (segment (start 55 14.5) (end 55 15.5) (width 0.25) (layer "F.Cu") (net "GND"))
 (segment (start 19 21.5) (end 18.9 21.5) (width 0.25) (layer "F.Cu") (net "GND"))
 (segment (start -1.965 22.04) (end -0.4 22.04) (width 0.25) (layer "F.Cu") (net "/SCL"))
 (via (at -0.4 22.04) (size 0.6) (drill 0.3) (layers "F.Cu" "B.Cu") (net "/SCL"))
 (segment (start 38 39) (end 38 40) (width 0.25) (layer "B.Cu") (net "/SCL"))
 (segment (start 38 14.25) (end 38 13) (width 0.25) (layer "B.Cu") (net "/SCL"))
 (segment (start 39.5 14.25) (end 38 14.25) (width 0.25) (layer "B.Cu") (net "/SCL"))
 (segment (start -1 19) (end -1 18.75) (width 0.25) (layer "B.Cu") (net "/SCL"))
 (segment (start 36.5 18.75) (end 36.5 27.25) (width 0.25) (layer "B.Cu") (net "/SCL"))
 (segment (start -0.4 22.04) (end -0.5 22) (width 0.25) (layer "B.Cu") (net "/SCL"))
 (segment (start -1 18.75) (end 36.5 18.75) (width 0.25) (layer "B.Cu") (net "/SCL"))
 (segment (start -0.5 22) (end -1.25 22) (width 0.25) (layer "B.Cu") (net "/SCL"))
 (segment (start 36.5 27.25) (end 36.5 39) (width 0.25) (layer "B.Cu") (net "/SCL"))
 (segment (start 38 13) (end 38 13.08) (width 0.25) (layer "B.Cu") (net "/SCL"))
 (segment (start 38 40) (end 38 40.08) (width 0.25) (layer "B.Cu") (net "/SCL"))
 (segment (start 36.5 27.25) (end 39.5 27.25) (width 0.25) (layer "B.Cu") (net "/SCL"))
 (segment (start -1.25 19) (end -1 19) (width 0.25) (layer "B.Cu") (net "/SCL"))
 (segment (start -1.25 22) (end -1.25 19) (width 0.25) (layer "B.Cu") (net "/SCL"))
 (segment (start 36.5 39) (end 38 39) (width 0.25) (layer "B.Cu") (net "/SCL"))
 (segment (start 39.5 27.25) (end 39.5 14.25) (width 0.25) (layer "B.Cu") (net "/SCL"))
 (segment (start -1.965 24.58) (end -0.4 24.58) (width 0.25) (layer "F.Cu") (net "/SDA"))
 (via (at -0.4 24.58) (size 0.6) (drill 0.3) (layers "F.Cu" "B.Cu") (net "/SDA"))
 (segment (start -2 18.75) (end -1.75 18.75) (width 0.25) (layer "B.Cu") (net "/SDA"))
 (segment (start -1 16.25) (end 17.25 16.25) (width 0.25) (layer "B.Cu") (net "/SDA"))
 (segment (start -1.5 18.25) (end -1.25 18.25) (width 0.25) (layer "B.Cu") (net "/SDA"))
 (segment (start -1 16.5) (end -1 16.25) (width 0.25) (layer "B.Cu") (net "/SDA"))
 (segment (start -1.75 18.75) (end -1.75 18.5) (width 0.25) (layer "B.Cu") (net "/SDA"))
 (segment (start 38 41.5) (end 38 42.5) (width 0.25) (layer "B.Cu") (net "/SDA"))
 (segment (start -0.5 24.5) (end 17.25 24.5) (width 0.25) (layer "B.Cu") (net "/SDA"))
 (segment (start 17.25 16.25) (end 17.25 15.5) (width 0.25) (layer "B.Cu") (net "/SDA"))
 (segment (start -0.4 24.58) (end -0.5 24.5) (width 0.25) (layer "B.Cu") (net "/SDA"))
 (segment (start 36.5 39.75) (end 36.5 41.5) (width 0.25) (layer "B.Cu") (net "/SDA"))
 (segment (start -1.75 18.5) (end -1.5 18.5) (width 0.25) (layer "B.Cu") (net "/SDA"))
 (segment (start -1.25 18.25) (end -1.25 16.5) (width 0.25) (layer "B.Cu") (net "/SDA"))
 (segment (start 17.25 15.5) (end 38 15.5) (width 0.25) (layer "B.Cu") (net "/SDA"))
 (segment (start 36.5 41.5) (end 38 41.5) (width 0.25) (layer "B.Cu") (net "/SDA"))
 (segment (start 36.25 39.75) (end 36.5 39.75) (width 0.25) (layer "B.Cu") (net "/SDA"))
 (segment (start 35.75 39.25) (end 36 39.25) (width 0.25) (layer "B.Cu") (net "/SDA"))
 (segment (start -0.5 24.5) (end -2 24.5) (width 0.25) (layer "B.Cu") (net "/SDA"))
 (segment (start -1.25 16.5) (end -1 16.5) (width 0.25) (layer "B.Cu") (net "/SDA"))
 (segment (start 38 15.5) (end 38 15.62) (width 0.25) (layer "B.Cu") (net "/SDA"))
 (segment (start 38 42.5) (end 38 42.62) (width 0.25) (layer "B.Cu") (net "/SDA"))
 (segment (start -2 24.5) (end -2 18.75) (width 0.25) (layer "B.Cu") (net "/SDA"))
 (segment (start 36 39.25) (end 36 39.5) (width 0.25) (layer "B.Cu") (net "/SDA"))
 (segment (start 36 39.5) (end 36.25 39.5) (width 0.25) (layer "B.Cu") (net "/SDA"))
 (segment (start 35.75 31.5) (end 35.75 39.25) (width 0.25) (layer "B.Cu") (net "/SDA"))
 (segment (start 36.25 39.5) (end 36.25 39.75) (width 0.25) (layer "B.Cu") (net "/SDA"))
 (segment (start 17.25 24.5) (end 17.25 31.5) (width 0.25) (layer "B.Cu") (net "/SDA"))
 (segment (start -1.5 18.5) (end -1.5 18.25) (width 0.25) (layer "B.Cu") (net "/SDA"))
 (segment (start 17.25 31.5) (end 35.75 31.5) (width 0.25) (layer "B.Cu") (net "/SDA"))
 (segment (start -1.965 14.42) (end -0.4 14.42) (width 0.25) (layer "F.Cu") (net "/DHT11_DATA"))
 (via (at -0.4 14.42) (size 0.6) (drill 0.3) (layers "F.Cu" "B.Cu") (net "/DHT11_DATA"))
 (segment (start -0.5 14.5) (end 36.5 14.5) (width 0.25) (layer "B.Cu") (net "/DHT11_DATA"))
 (segment (start 36.5 6.5) (end 53.75 6.5) (width 0.25) (layer "B.Cu") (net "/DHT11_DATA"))
 (segment (start -0.4 14.42) (end -0.5 14.5) (width 0.25) (layer "B.Cu") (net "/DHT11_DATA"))
 (segment (start 53.75 6.5) (end 53.75 9.25) (width 0.25) (layer "B.Cu") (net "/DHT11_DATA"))
 (segment (start 53.75 9.25) (end 55 9.25) (width 0.25) (layer "B.Cu") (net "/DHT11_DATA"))
 (segment (start 36.5 14.5) (end 36.5 6.5) (width 0.25) (layer "B.Cu") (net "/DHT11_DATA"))
 (segment (start 55 9.25) (end 55 10.5) (width 0.25) (layer "B.Cu") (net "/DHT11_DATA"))
 (segment (start 55 10.5) (end 55 10.54) (width 0.25) (layer "B.Cu") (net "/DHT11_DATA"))
 (segment (start -1.965 16.96) (end -0.4 16.96) (width 0.25) (layer "F.Cu") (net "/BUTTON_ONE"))
 (via (at -0.4 16.96) (size 0.6) (drill 0.3) (layers "F.Cu" "B.Cu") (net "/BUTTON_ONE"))
 (segment (start -0.5 17) (end 19 17) (width 0.25) (layer "B.Cu") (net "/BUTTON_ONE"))
 (segment (start 25.5 17) (end 25.4 17) (width 0.25) (layer "B.Cu") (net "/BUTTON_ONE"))
 (segment (start 19 17) (end 25.5 17) (width 0.25) (layer "B.Cu") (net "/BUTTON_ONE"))
 (segment (start 19 17) (end 18.9 17) (width 0.25) (layer "B.Cu") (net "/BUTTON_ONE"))
 (segment (start -0.4 16.96) (end -0.5 17) (width 0.25) (layer "B.Cu") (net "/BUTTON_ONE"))
 (segment (start -1.965 19.5) (end -0.4 19.5) (width 0.25) (layer "F.Cu") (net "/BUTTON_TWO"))
 (via (at -0.4 19.5) (size 0.6) (drill 0.3) (layers "F.Cu" "B.Cu") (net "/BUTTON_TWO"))
 (segment (start 25.5 30) (end 25.4 30) (width 0.25) (layer "B.Cu") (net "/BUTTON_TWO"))
 (segment (start -0.5 19.5) (end 17.25 19.5) (width 0.25) (layer "B.Cu") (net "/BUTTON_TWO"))
 (segment (start 19 30) (end 25.5 30) (width 0.25) (layer "B.Cu") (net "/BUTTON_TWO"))
 (segment (start 17.25 23) (end 19 23) (width 0.25) (layer "B.Cu") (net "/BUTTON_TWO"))
 (segment (start 19 23) (end 19 30) (width 0.25) (layer "B.Cu") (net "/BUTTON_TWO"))
 (segment (start -0.4 19.5) (end -0.5 19.5) (width 0.25) (layer "B.Cu") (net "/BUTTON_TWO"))
 (segment (start 19 30) (end 18.9 30) (width 0.25) (layer "B.Cu") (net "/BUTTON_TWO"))
 (segment (start 17.25 19.5) (end 17.25 23) (width 0.25) (layer "B.Cu") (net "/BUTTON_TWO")))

